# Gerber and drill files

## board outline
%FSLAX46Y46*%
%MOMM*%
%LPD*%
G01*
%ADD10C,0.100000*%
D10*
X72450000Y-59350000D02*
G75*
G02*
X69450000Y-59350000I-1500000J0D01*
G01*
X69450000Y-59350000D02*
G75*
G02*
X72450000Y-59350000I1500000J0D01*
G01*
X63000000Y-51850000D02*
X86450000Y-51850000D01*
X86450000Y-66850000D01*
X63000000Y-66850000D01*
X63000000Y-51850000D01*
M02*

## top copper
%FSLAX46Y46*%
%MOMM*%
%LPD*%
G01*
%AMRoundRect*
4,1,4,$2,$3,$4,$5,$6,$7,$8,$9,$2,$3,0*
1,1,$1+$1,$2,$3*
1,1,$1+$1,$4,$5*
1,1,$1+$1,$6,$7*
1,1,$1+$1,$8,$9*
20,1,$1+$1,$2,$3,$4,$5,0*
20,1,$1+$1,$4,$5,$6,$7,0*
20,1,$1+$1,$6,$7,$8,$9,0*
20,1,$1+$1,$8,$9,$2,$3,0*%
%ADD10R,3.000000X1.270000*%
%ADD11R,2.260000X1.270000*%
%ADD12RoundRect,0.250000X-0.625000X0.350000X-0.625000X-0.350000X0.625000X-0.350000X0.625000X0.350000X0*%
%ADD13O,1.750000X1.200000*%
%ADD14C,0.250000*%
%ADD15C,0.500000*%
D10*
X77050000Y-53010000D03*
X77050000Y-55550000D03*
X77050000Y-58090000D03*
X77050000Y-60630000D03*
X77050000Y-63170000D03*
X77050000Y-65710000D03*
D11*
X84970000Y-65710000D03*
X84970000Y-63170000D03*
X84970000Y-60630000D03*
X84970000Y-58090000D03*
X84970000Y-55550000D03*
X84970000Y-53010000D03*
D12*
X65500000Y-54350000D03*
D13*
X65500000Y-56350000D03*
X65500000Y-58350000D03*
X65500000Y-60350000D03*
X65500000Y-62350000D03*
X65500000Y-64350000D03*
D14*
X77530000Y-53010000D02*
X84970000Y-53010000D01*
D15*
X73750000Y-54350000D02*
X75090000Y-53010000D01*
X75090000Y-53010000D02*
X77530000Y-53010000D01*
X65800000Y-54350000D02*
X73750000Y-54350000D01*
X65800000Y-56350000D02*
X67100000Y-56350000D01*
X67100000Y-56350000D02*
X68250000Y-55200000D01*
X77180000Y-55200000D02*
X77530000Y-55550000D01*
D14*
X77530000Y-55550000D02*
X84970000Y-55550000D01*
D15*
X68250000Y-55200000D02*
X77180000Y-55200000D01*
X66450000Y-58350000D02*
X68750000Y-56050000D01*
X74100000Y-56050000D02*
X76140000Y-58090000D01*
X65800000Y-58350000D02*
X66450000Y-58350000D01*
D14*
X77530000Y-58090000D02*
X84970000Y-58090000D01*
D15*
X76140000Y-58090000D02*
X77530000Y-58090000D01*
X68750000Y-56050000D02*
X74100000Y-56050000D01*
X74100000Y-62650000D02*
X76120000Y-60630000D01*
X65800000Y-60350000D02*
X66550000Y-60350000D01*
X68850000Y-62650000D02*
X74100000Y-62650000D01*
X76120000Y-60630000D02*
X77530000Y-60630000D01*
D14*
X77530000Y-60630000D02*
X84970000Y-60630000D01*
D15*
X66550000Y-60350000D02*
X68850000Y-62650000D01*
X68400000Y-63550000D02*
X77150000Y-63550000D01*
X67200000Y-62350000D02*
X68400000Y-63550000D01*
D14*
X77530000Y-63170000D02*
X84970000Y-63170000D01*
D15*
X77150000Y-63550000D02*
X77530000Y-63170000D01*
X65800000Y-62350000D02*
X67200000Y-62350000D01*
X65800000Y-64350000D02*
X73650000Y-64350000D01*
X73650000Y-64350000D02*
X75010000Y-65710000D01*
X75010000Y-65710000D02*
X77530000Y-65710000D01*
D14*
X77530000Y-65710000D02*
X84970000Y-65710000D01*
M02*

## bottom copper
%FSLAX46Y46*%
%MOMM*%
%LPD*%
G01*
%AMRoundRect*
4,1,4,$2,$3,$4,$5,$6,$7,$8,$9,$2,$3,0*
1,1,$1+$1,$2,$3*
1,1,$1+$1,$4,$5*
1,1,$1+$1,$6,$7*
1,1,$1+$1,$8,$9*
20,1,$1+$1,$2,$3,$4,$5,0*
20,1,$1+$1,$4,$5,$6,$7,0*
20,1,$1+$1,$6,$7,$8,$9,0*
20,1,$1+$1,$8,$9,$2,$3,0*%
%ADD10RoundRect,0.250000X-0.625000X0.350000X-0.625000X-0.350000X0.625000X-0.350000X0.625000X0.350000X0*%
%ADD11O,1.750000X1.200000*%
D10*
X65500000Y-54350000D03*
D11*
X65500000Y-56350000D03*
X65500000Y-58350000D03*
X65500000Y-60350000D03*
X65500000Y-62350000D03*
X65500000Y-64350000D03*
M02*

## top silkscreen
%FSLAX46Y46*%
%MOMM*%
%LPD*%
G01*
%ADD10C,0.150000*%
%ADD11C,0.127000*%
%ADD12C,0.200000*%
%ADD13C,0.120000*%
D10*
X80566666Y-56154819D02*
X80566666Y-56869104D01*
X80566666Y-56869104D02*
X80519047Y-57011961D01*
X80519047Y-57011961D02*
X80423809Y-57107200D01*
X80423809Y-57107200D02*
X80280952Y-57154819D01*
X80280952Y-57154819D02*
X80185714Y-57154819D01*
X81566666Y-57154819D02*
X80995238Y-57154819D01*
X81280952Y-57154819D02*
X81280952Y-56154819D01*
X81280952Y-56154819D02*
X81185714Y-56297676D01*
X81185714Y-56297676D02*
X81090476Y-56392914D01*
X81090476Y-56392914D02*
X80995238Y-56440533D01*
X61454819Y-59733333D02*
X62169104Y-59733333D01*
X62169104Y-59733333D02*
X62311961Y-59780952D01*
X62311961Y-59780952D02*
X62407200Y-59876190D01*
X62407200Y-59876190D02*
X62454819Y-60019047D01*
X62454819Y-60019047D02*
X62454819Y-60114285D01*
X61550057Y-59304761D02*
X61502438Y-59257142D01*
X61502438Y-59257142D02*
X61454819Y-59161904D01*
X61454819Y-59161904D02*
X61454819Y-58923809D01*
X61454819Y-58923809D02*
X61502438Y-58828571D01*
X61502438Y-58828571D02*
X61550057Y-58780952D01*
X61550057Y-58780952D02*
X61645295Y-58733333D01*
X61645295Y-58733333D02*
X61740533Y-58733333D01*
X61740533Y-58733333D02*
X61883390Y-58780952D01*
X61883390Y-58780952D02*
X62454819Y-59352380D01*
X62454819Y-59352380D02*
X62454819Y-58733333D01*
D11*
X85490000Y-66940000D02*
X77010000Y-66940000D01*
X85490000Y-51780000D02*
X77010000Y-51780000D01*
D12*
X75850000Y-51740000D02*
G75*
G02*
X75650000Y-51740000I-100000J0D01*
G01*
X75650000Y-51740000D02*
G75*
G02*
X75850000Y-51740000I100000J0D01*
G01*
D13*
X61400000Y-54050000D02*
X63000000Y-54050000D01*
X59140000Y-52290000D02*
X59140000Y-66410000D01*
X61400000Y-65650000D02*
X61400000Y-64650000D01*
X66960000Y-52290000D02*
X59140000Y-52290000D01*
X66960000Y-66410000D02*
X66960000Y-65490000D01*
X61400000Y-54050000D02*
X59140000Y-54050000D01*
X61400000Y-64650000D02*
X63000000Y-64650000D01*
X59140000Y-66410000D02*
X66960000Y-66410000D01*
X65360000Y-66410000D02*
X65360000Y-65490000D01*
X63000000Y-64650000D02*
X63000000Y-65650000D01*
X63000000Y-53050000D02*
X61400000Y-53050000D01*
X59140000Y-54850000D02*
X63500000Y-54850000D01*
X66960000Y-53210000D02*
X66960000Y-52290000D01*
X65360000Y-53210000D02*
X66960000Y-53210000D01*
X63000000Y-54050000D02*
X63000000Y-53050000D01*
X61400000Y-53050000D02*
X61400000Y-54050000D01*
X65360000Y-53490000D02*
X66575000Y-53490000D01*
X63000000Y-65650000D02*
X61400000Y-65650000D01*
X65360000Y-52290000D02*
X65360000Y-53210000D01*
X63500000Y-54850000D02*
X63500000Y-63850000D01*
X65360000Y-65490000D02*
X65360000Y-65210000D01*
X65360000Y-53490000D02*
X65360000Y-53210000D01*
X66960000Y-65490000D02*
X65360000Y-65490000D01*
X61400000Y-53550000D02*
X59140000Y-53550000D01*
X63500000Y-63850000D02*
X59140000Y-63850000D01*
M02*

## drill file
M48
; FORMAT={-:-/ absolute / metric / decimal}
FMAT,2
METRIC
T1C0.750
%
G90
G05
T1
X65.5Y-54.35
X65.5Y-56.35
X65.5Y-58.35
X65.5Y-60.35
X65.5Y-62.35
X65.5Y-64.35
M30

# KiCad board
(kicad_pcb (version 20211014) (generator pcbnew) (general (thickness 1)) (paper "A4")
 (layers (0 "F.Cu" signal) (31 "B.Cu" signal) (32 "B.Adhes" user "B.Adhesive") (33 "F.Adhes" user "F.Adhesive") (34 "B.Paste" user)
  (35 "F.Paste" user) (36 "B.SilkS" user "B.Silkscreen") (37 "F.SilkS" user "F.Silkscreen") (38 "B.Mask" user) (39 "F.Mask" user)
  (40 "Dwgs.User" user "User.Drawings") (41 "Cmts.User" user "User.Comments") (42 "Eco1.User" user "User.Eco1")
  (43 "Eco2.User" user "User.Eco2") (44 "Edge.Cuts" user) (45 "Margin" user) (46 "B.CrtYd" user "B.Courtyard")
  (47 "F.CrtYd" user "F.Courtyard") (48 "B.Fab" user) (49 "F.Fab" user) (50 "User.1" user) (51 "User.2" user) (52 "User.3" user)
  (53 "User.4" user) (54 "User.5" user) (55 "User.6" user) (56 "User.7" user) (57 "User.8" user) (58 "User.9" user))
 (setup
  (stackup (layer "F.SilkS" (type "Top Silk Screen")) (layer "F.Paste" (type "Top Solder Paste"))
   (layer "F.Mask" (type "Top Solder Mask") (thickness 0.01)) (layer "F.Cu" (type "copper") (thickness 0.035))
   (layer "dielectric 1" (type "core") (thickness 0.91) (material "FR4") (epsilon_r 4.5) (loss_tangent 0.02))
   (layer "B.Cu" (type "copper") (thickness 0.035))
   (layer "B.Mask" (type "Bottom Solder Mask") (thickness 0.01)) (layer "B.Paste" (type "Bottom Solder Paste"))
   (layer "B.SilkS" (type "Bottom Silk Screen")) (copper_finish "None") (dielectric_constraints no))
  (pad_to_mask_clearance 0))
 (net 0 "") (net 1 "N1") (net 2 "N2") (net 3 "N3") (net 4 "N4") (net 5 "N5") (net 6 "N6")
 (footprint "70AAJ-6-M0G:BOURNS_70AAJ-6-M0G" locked (layer "F.Cu") (at 81.25 59.36)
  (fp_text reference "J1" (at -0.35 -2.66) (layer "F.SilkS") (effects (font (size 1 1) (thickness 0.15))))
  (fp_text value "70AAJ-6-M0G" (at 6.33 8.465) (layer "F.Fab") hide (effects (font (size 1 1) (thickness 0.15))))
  (fp_line (start 4.24 7.58) (end -4.24 7.58) (layer "F.SilkS") (width 0.127))
  (fp_line (start 4.24 -7.58) (end -4.24 -7.58) (layer "F.SilkS") (width 0.127))
  (fp_circle (center -5.5 -7.62) (end -5.4 -7.62) (layer "F.SilkS") (width 0.2) (fill none))
  (pad "1" smd rect locked (at -4.2 -6.35) (size 3 1.27) (layers "F.Cu" "F.Paste" "F.Mask") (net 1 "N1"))
  (pad "2" smd rect locked (at -4.2 -3.81) (size 3 1.27) (layers "F.Cu" "F.Paste" "F.Mask") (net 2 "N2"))
  (pad "3" smd rect locked (at -4.2 -1.27) (size 3 1.27) (layers "F.Cu" "F.Paste" "F.Mask") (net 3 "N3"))
  (pad "4" smd rect locked (at -4.2 1.27) (size 3 1.27) (layers "F.Cu" "F.Paste" "F.Mask") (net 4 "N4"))
  (pad "5" smd rect locked (at -4.2 3.81) (size 3 1.27) (layers "F.Cu" "F.Paste" "F.Mask") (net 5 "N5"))
  (pad "6" smd rect locked (at -4.2 6.35) (size 3 1.27) (layers "F.Cu" "F.Paste" "F.Mask") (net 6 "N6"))
  (pad "7" smd rect locked (at 3.72 6.35) (size 2.26 1.27) (layers "F.Cu" "F.Paste" "F.Mask") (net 6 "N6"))
  (pad "8" smd rect locked (at 3.72 3.81) (size 2.26 1.27) (layers "F.Cu" "F.Paste" "F.Mask") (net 5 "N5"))
  (pad "9" smd rect locked (at 3.72 1.27) (size 2.26 1.27) (layers "F.Cu" "F.Paste" "F.Mask") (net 4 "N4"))
  (pad "10" smd rect locked (at 3.72 -1.27) (size 2.26 1.27) (layers "F.Cu" "F.Paste" "F.Mask") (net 3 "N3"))
  (pad "11" smd rect locked (at 3.72 -3.81) (size 2.26 1.27) (layers "F.Cu" "F.Paste" "F.Mask") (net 2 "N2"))
  (pad "12" smd rect locked (at 3.72 -6.35) (size 2.26 1.27) (layers "F.Cu" "F.Paste" "F.Mask") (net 1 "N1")))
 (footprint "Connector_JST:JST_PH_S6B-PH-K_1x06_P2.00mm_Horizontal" (layer "F.Cu") (at 65.5 54.35 -90)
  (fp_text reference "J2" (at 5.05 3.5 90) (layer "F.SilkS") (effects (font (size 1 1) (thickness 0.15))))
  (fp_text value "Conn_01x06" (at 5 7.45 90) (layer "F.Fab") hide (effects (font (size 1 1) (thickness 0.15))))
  (fp_line (start -0.3 4.1) (end -0.3 2.5) (layer "F.SilkS") (width 0.12))
  (fp_line (start -2.06 6.36) (end 12.06 6.36) (layer "F.SilkS") (width 0.12))
  (fp_line (start 11.3 4.1) (end 10.3 4.1) (layer "F.SilkS") (width 0.12))
  (fp_line (start -2.06 -1.46) (end -2.06 6.36) (layer "F.SilkS") (width 0.12))
  (fp_line (start 12.06 -1.46) (end 11.14 -1.46) (layer "F.SilkS") (width 0.12))
  (fp_line (start -0.3 4.1) (end -0.3 6.36) (layer "F.SilkS") (width 0.12))
  (fp_line (start 10.3 4.1) (end 10.3 2.5) (layer "F.SilkS") (width 0.12))
  (fp_line (start 12.06 6.36) (end 12.06 -1.46) (layer "F.SilkS") (width 0.12))
  (fp_line (start 12.06 0.14) (end 11.14 0.14) (layer "F.SilkS") (width 0.12))
  (fp_line (start 10.3 2.5) (end 11.3 2.5) (layer "F.SilkS") (width 0.12))
  (fp_line (start -1.3 2.5) (end -1.3 4.1) (layer "F.SilkS") (width 0.12))
  (fp_line (start 0.5 6.36) (end 0.5 2) (layer "F.SilkS") (width 0.12))
  (fp_line (start -1.14 -1.46) (end -2.06 -1.46) (layer "F.SilkS") (width 0.12))
  (fp_line (start -1.14 0.14) (end -1.14 -1.46) (layer "F.SilkS") (width 0.12))
  (fp_line (start -0.3 2.5) (end -1.3 2.5) (layer "F.SilkS") (width 0.12))
  (fp_line (start -1.3 4.1) (end -0.3 4.1) (layer "F.SilkS") (width 0.12))
  (fp_line (start -0.86 0.14) (end -0.86 -1.075) (layer "F.SilkS") (width 0.12))
  (fp_line (start 11.3 2.5) (end 11.3 4.1) (layer "F.SilkS") (width 0.12))
  (fp_line (start -2.06 0.14) (end -1.14 0.14) (layer "F.SilkS") (width 0.12))
  (fp_line (start 0.5 2) (end 9.5 2) (layer "F.SilkS") (width 0.12))
  (fp_line (start 11.14 0.14) (end 10.86 0.14) (layer "F.SilkS") (width 0.12))
  (fp_line (start -0.86 0.14) (end -1.14 0.14) (layer "F.SilkS") (width 0.12))
  (fp_line (start 11.14 -1.46) (end 11.14 0.14) (layer "F.SilkS") (width 0.12))
  (fp_line (start -0.8 4.1) (end -0.8 6.36) (layer "F.SilkS") (width 0.12))
  (fp_line (start 9.5 2) (end 9.5 6.36) (layer "F.SilkS") (width 0.12))
  (pad "1" thru_hole roundrect (at 0 0 270) (size 1.2 1.75) (drill 0.75) (layers *.Cu *.Mask) (roundrect_rratio 0.208333) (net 1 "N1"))
  (pad "2" thru_hole oval (at 2 0 270) (size 1.2 1.75) (drill 0.75) (layers *.Cu *.Mask) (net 2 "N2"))
  (pad "3" thru_hole oval (at 4 0 270) (size 1.2 1.75) (drill 0.75) (layers *.Cu *.Mask) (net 3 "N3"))
  (pad "4" thru_hole oval (at 6 0 270) (size 1.2 1.75) (drill 0.75) (layers *.Cu *.Mask) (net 4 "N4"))
  (pad "5" thru_hole oval (at 8 0 270) (size 1.2 1.75) (drill 0.75) (layers *.Cu *.Mask) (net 5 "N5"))
  (pad "6" thru_hole oval (at 10 0 270) (size 1.2 1.75) (drill 0.75) (layers *.Cu *.Mask) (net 6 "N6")))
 (gr_circle locked (center 70.95 59.35) (end 72.45 59.35) (layer "Edge.Cuts") (width 0.1) (fill none))
 (gr_rect locked (start 63 51.85) (end 86.45 66.85) (layer "Edge.Cuts") (width 0.1) (fill none))
 (segment (start 77.53 53.01) (end 84.97 53.01) (width 0.25) (layer "F.Cu") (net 1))
 (segment (start 73.75 54.35) (end 75.09 53.01) (width 0.5) (layer "F.Cu") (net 1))
 (segment (start 75.09 53.01) (end 77.53 53.01) (width 0.5) (layer "F.Cu") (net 1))
 (segment (start 65.8 54.35) (end 73.75 54.35) (width 0.5) (layer "F.Cu") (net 1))
 (segment (start 65.8 56.35) (end 67.1 56.35) (width 0.5) (layer "F.Cu") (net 2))
 (segment (start 67.1 56.35) (end 68.25 55.2) (width 0.5) (layer "F.Cu") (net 2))
 (segment (start 77.18 55.2) (end 77.53 55.55) (width 0.5) (layer "F.Cu") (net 2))
 (segment (start 77.53 55.55) (end 84.97 55.55) (width 0.25) (layer "F.Cu") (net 2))
 (segment (start 68.25 55.2) (end 77.18 55.2) (width 0.5) (layer "F.Cu") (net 2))
 (segment (start 66.45 58.35) (end 68.75 56.05) (width 0.5) (layer "F.Cu") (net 3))
 (segment (start 74.1 56.05) (end 76.14 58.09) (width 0.5) (layer "F.Cu") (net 3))
 (segment (start 65.8 58.35) (end 66.45 58.35) (width 0.5) (layer "F.Cu") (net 3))
 (segment (start 77.53 58.09) (end 84.97 58.09) (width 0.25) (layer "F.Cu") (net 3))
 (segment (start 76.14 58.09) (end 77.53 58.09) (width 0.5) (layer "F.Cu") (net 3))
 (segment (start 68.75 56.05) (end 74.1 56.05) (width 0.5) (layer "F.Cu") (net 3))
 (segment (start 74.1 62.65) (end 76.12 60.63) (width 0.5) (layer "F.Cu") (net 4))
 (segment (start 65.8 60.35) (end 66.55 60.35) (width 0.5) (layer "F.Cu") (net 4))
 (segment (start 68.85 62.65) (end 74.1 62.65) (width 0.5) (layer "F.Cu") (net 4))
 (segment (start 76.12 60.63) (end 77.53 60.63) (width 0.5) (layer "F.Cu") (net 4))
 (segment (start 77.53 60.63) (end 84.97 60.63) (width 0.25) (layer "F.Cu") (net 4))
 (segment (start 66.55 60.35) (end 68.85 62.65) (width 0.5) (layer "F.Cu") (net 4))
 (segment (start 68.4 63.55) (end 77.15 63.55) (width 0.5) (layer "F.Cu") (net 5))
 (segment (start 67.2 62.35) (end 68.4 63.55) (width 0.5) (layer "F.Cu") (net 5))
 (segment (start 77.53 63.17) (end 84.97 63.17) (width 0.25) (layer "F.Cu") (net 5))
 (segment (start 77.15 63.55) (end 77.53 63.17) (width 0.5) (layer "F.Cu") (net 5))
 (segment (start 65.8 62.35) (end 67.2 62.35) (width 0.5) (layer "F.Cu") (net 5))
 (segment (start 65.8 64.35) (end 73.65 64.35) (width 0.5) (layer "F.Cu") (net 6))
 (segment (start 73.65 64.35) (end 75.01 65.71) (width 0.5) (layer "F.Cu") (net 6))
 (segment (start 75.01 65.71) (end 77.53 65.71) (width 0.5) (layer "F.Cu") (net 6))
 (segment (start 77.53 65.71) (end 84.97 65.71) (width 0.25) (layer "F.Cu") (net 6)))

